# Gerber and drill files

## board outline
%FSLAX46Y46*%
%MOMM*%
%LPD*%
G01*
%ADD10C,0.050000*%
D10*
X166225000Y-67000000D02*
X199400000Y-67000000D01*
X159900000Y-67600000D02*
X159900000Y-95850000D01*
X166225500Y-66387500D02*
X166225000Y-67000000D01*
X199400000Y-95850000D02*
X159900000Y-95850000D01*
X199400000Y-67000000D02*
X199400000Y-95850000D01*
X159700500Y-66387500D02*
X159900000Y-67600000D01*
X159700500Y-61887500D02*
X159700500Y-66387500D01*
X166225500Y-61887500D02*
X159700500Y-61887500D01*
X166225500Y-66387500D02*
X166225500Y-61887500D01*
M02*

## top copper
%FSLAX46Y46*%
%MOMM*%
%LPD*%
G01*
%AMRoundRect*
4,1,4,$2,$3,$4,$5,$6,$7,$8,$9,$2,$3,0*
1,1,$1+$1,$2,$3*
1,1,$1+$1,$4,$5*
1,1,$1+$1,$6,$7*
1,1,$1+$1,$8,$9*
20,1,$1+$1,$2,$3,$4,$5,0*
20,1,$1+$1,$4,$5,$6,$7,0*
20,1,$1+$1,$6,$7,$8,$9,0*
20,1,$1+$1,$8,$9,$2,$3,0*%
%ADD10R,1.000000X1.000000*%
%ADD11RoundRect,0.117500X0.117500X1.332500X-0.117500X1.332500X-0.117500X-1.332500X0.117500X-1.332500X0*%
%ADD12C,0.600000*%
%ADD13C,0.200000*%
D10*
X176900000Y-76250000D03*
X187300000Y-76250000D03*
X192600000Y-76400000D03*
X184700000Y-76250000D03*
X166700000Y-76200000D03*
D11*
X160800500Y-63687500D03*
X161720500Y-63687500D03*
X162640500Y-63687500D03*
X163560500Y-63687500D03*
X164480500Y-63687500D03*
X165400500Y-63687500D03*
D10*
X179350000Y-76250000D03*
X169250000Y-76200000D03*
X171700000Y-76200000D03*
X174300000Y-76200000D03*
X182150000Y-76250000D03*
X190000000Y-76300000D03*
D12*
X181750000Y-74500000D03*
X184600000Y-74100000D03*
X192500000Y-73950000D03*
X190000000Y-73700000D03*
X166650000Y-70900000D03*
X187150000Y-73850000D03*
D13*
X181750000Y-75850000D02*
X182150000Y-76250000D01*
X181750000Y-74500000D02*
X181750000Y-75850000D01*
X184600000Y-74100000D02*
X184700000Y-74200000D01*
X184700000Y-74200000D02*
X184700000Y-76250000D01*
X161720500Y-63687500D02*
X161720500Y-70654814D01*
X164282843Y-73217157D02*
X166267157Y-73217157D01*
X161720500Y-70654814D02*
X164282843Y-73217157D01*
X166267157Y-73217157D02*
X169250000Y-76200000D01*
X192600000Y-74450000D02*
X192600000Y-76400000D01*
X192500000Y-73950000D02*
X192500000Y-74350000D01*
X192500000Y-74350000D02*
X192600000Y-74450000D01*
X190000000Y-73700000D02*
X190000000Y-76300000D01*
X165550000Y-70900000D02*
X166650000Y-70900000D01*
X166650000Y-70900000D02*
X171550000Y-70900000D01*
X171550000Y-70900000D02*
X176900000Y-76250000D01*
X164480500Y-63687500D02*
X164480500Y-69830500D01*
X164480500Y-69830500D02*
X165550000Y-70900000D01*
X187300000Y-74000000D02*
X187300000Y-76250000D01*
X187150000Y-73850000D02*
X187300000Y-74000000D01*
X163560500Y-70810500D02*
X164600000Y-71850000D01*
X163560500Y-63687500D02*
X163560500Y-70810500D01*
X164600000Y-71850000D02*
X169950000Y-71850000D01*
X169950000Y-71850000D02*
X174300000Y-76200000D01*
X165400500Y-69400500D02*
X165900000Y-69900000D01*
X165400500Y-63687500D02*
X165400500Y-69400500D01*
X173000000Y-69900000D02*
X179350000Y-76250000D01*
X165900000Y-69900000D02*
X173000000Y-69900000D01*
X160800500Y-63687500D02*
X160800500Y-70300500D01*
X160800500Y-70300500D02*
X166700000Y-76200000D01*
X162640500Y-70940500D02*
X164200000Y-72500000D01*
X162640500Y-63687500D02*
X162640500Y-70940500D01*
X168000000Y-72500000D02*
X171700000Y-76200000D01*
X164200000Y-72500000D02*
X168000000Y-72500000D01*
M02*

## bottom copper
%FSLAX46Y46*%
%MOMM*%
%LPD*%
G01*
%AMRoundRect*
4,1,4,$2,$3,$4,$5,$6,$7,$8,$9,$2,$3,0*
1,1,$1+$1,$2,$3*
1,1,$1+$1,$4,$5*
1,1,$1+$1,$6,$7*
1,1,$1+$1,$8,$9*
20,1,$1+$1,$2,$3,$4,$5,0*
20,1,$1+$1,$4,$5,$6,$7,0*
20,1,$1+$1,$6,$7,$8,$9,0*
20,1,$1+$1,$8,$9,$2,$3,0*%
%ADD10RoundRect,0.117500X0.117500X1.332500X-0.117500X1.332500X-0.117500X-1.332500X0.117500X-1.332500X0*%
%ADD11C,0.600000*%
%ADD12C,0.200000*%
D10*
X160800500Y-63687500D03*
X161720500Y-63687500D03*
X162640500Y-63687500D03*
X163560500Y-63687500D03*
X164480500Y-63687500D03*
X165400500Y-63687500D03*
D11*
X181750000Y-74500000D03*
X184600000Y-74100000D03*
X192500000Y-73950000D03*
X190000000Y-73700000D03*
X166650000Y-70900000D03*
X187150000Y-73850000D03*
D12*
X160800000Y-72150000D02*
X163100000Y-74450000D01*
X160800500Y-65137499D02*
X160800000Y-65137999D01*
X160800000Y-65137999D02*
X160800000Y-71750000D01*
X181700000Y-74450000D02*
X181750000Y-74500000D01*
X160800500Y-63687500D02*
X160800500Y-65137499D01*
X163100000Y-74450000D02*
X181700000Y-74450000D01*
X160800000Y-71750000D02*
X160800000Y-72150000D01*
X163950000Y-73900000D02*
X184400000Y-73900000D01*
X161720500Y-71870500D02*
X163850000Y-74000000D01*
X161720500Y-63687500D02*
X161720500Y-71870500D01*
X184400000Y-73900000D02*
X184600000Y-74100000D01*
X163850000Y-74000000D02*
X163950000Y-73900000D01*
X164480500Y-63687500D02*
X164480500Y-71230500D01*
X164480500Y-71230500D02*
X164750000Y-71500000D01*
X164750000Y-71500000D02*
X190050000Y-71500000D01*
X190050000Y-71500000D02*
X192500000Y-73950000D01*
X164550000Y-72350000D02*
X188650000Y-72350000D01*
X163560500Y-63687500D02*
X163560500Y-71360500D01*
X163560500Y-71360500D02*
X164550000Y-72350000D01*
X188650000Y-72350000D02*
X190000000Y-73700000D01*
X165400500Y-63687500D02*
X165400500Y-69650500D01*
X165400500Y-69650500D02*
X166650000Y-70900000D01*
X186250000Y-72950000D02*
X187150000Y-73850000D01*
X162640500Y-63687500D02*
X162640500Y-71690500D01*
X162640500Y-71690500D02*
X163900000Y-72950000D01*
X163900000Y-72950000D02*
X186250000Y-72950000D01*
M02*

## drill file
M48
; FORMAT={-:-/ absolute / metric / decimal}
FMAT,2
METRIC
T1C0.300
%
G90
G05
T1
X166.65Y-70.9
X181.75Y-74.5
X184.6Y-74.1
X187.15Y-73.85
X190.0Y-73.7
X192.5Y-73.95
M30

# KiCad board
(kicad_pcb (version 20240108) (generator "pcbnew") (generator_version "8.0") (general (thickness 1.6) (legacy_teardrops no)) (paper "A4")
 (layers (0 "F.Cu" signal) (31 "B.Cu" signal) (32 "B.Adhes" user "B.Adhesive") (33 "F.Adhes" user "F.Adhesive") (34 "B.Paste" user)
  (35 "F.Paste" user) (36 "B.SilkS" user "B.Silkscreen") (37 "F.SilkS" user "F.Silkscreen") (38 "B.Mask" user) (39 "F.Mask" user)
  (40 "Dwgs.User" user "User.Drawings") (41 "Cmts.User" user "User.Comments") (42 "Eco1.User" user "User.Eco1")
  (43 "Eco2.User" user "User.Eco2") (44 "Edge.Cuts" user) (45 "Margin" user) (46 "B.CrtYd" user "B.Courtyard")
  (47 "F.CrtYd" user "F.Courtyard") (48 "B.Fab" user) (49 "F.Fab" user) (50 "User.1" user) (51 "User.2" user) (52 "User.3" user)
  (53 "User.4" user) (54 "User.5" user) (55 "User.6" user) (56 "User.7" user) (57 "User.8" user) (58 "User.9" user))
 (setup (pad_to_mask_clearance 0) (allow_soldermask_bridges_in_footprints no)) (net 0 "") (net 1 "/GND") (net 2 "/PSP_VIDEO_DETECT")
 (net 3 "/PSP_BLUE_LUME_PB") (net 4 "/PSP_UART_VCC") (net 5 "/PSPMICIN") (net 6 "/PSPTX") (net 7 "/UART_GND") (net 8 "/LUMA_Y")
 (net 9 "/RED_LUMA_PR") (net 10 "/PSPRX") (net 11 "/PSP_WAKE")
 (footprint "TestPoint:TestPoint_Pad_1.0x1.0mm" (layer "F.Cu") (at 176.9 76.25)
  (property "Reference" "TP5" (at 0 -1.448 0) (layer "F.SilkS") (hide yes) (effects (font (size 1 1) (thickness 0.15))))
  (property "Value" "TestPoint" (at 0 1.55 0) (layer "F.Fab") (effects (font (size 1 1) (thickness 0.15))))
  (pad "1" smd rect (at 0 0) (size 1 1) (layers "F.Cu" "F.Mask") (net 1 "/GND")))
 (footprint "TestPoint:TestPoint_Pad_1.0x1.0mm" (layer "F.Cu") (at 187.3 76.25)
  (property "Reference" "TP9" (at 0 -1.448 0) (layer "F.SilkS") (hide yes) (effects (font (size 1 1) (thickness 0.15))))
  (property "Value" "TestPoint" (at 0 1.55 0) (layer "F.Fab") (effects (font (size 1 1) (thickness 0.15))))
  (pad "1" smd rect (at 0 0) (size 1 1) (layers "F.Cu" "F.Mask") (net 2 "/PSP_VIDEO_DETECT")))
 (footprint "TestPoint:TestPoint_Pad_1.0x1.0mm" (layer "F.Cu") (at 192.6 76.4)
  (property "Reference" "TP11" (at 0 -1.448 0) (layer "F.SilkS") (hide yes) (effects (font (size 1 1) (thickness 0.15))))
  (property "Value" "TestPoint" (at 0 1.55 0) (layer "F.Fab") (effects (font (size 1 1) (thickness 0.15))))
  (pad "1" smd rect (at 0 0) (size 1 1) (layers "F.Cu" "F.Mask") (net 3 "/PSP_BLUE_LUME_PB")))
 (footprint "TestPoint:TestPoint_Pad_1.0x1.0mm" (layer "F.Cu") (at 184.7 76.25)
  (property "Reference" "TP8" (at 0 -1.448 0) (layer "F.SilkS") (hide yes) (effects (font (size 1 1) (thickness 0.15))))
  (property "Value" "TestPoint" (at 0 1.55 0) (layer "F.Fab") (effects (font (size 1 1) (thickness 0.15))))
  (pad "1" smd rect (at 0 0) (size 1 1) (layers "F.Cu" "F.Mask") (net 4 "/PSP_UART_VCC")))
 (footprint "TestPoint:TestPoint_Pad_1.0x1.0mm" (layer "F.Cu") (at 166.7 76.2)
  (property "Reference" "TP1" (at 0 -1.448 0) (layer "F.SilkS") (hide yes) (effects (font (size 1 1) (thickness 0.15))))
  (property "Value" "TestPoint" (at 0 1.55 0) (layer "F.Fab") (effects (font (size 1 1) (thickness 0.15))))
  (pad "1" smd rect (at 0 0) (size 1 1) (layers "F.Cu" "F.Mask") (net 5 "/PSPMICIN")))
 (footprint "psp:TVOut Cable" (layer "F.Cu") (at 168.8255 70.9875)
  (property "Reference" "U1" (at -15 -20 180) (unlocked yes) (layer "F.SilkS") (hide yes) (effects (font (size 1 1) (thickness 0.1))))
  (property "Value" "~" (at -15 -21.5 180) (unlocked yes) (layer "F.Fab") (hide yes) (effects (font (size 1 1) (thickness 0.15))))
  (fp_line (start -9.125 -9.1) (end -9.125 -4.6) (stroke (width 0.05) (type default)) (layer "Edge.Cuts"))
  (fp_line (start -2.6 -9.1) (end -9.125 -9.1) (stroke (width 0.05) (type default)) (layer "Edge.Cuts"))
  (fp_line (start -2.6 -4.6) (end -2.6 -9.1) (stroke (width 0.05) (type default)) (layer "Edge.Cuts"))
  (pad "1" smd roundrect (at -8.025 -7.3 180) (size 0.47 2.9) (layers "F.Cu" "F.Paste" "F.Mask") (roundrect_rratio 0.25) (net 5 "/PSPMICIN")
   (thermal_bridge_angle 45))
  (pad "2" smd roundrect (at -7.105 -7.3 180) (size 0.47 2.9) (layers "F.Cu" "F.Paste" "F.Mask") (roundrect_rratio 0.25) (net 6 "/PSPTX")
   (thermal_bridge_angle 45))
  (pad "3" smd roundrect (at -6.185 -7.3 180) (size 0.47 2.9) (layers "F.Cu" "F.Paste" "F.Mask") (roundrect_rratio 0.25) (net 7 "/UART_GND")
   (thermal_bridge_angle 45))
  (pad "4" smd roundrect (at -5.265 -7.3 180) (size 0.47 2.9) (layers "F.Cu" "F.Paste" "F.Mask") (roundrect_rratio 0.25) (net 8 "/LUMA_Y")
   (thermal_bridge_angle 45))
  (pad "5" smd roundrect (at -4.345 -7.3 180) (size 0.47 2.9) (layers "F.Cu" "F.Paste" "F.Mask") (roundrect_rratio 0.25) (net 1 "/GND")
   (thermal_bridge_angle 45))
  (pad "6" smd roundrect (at -3.425 -7.3 180) (size 0.47 2.9) (layers "F.Cu" "F.Paste" "F.Mask") (roundrect_rratio 0.25)
   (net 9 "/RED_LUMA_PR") (thermal_bridge_angle 45))
  (pad "7" smd roundrect (at -8.025 -7.3 180) (size 0.47 2.9) (layers "B.Cu" "B.Paste" "B.Mask") (roundrect_rratio 0.25) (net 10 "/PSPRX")
   (thermal_bridge_angle 45))
  (pad "8" smd roundrect (at -7.105 -7.3 180) (size 0.47 2.9) (layers "B.Cu" "B.Paste" "B.Mask") (roundrect_rratio 0.25)
   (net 4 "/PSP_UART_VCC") (thermal_bridge_angle 45))
  (pad "9" smd roundrect (at -6.185 -7.3 180) (size 0.47 2.9) (layers "B.Cu" "B.Paste" "B.Mask") (roundrect_rratio 0.25)
   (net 2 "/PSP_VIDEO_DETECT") (thermal_bridge_angle 45))
  (pad "10" smd roundrect (at -5.265 -7.3 180) (size 0.47 2.9) (layers "B.Cu" "B.Paste" "B.Mask") (roundrect_rratio 0.25)
   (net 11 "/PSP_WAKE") (thermal_bridge_angle 45))
  (pad "11" smd roundrect (at -4.345 -7.3 180) (size 0.47 2.9) (layers "B.Cu" "B.Paste" "B.Mask") (roundrect_rratio 0.25)
   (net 3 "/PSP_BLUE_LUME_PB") (thermal_bridge_angle 45))
  (pad "12" smd roundrect (at -3.425 -7.3 180) (size 0.47 2.9) (layers "B.Cu" "B.Paste" "B.Mask") (roundrect_rratio 0.25) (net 1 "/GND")
   (thermal_bridge_angle 45)))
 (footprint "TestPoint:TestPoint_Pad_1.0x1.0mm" (layer "F.Cu") (at 179.35 76.25)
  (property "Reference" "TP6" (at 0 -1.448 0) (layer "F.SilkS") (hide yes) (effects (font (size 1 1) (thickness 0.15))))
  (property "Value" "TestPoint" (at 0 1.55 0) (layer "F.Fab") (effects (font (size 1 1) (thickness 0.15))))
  (pad "1" smd rect (at 0 0) (size 1 1) (layers "F.Cu" "F.Mask") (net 9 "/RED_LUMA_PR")))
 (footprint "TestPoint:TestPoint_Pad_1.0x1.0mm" (layer "F.Cu") (at 169.25 76.2)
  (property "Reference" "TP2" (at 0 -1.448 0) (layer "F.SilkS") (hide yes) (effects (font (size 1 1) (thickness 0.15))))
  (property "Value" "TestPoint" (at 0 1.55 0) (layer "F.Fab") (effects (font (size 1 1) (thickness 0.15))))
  (pad "1" smd rect (at 0 0) (size 1 1) (layers "F.Cu" "F.Mask") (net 6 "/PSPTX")))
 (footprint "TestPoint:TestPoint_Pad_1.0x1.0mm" (layer "F.Cu") (at 171.7 76.2)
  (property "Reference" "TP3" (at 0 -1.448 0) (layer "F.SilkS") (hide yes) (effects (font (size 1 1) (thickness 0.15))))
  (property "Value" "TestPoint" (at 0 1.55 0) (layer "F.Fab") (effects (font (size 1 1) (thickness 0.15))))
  (pad "1" smd rect (at 0 0) (size 1 1) (layers "F.Cu" "F.Mask") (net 7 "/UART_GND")))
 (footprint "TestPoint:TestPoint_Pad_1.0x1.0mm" (layer "F.Cu") (at 174.3 76.2)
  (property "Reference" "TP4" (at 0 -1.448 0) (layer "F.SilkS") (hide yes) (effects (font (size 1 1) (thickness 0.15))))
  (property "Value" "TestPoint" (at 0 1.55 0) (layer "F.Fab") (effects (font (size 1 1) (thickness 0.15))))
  (pad "1" smd rect (at 0 0) (size 1 1) (layers "F.Cu" "F.Mask") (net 8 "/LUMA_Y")))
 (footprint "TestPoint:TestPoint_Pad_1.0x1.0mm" (layer "F.Cu") (at 182.15 76.25)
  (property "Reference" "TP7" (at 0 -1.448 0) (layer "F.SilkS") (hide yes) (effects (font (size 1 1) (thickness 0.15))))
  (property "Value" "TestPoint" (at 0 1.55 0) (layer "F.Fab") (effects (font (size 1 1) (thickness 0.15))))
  (pad "1" smd rect (at 0 0) (size 1 1) (layers "F.Cu" "F.Mask") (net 10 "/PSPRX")))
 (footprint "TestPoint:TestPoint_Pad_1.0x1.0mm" (layer "F.Cu") (at 190 76.3)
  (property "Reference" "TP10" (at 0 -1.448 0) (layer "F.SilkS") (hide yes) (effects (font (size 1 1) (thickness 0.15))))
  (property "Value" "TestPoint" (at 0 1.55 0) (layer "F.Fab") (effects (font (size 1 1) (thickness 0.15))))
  (pad "1" smd rect (at 0 0) (size 1 1) (layers "F.Cu" "F.Mask") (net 11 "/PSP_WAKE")))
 (gr_line (start 166.225 67) (end 199.4 67) (stroke (width 0.05) (type default)) (layer "Edge.Cuts"))
 (gr_line (start 159.9 67.6) (end 159.9 95.85) (stroke (width 0.05) (type default)) (layer "Edge.Cuts"))
 (gr_line (start 166.2255 66.3875) (end 166.225 67) (stroke (width 0.05) (type default)) (layer "Edge.Cuts"))
 (gr_line (start 199.4 95.85) (end 159.9 95.85) (stroke (width 0.05) (type default)) (layer "Edge.Cuts"))
 (gr_line (start 199.4 67) (end 199.4 95.85) (stroke (width 0.05) (type default)) (layer "Edge.Cuts"))
 (gr_line (start 159.7005 66.3875) (end 159.9 67.6) (stroke (width 0.05) (type default)) (layer "Edge.Cuts"))
 (segment (start 181.75 75.85) (end 182.15 76.25) (width 0.2) (layer "F.Cu") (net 10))
 (segment (start 181.75 74.5) (end 181.75 75.85) (width 0.2) (layer "F.Cu") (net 10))
 (via (at 181.75 74.5) (size 0.6) (drill 0.3) (layers "F.Cu" "B.Cu") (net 10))
 (segment (start 160.8 72.15) (end 163.1 74.45) (width 0.2) (layer "B.Cu") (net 10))
 (segment (start 160.8005 65.137499) (end 160.8 65.137999) (width 0.2) (layer "B.Cu") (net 10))
 (segment (start 160.8 65.137999) (end 160.8 71.75) (width 0.2) (layer "B.Cu") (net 10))
 (segment (start 181.7 74.45) (end 181.75 74.5) (width 0.2) (layer "B.Cu") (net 10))
 (segment (start 160.8005 63.6875) (end 160.8005 65.137499) (width 0.2) (layer "B.Cu") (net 10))
 (segment (start 163.1 74.45) (end 181.7 74.45) (width 0.2) (layer "B.Cu") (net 10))
 (segment (start 160.8 71.75) (end 160.8 72.15) (width 0.2) (layer "B.Cu") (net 10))
 (segment (start 184.6 74.1) (end 184.7 74.2) (width 0.2) (layer "F.Cu") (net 4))
 (segment (start 184.7 74.2) (end 184.7 76.25) (width 0.2) (layer "F.Cu") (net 4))
 (via (at 184.6 74.1) (size 0.6) (drill 0.3) (layers "F.Cu" "B.Cu") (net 4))
 (segment (start 163.95 73.9) (end 184.4 73.9) (width 0.2) (layer "B.Cu") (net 4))
 (segment (start 161.7205 71.8705) (end 163.85 74) (width 0.2) (layer "B.Cu") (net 4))
 (segment (start 161.7205 63.6875) (end 161.7205 71.8705) (width 0.2) (layer "B.Cu") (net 4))
 (segment (start 184.4 73.9) (end 184.6 74.1) (width 0.2) (layer "B.Cu") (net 4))
 (segment (start 163.85 74) (end 163.95 73.9) (width 0.2) (layer "B.Cu") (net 4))
 (segment (start 161.7205 63.6875) (end 161.7205 70.654814) (width 0.2) (layer "F.Cu") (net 6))
 (segment (start 164.282843 73.217157) (end 166.267157 73.217157) (width 0.2) (layer "F.Cu") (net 6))
 (segment (start 161.7205 70.654814) (end 164.282843 73.217157) (width 0.2) (layer "F.Cu") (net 6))
 (segment (start 166.267157 73.217157) (end 169.25 76.2) (width 0.2) (layer "F.Cu") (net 6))
 (segment (start 192.6 74.45) (end 192.6 76.4) (width 0.2) (layer "F.Cu") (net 3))
 (segment (start 192.5 73.95) (end 192.5 74.35) (width 0.2) (layer "F.Cu") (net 3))
 (segment (start 192.5 74.35) (end 192.6 74.45) (width 0.2) (layer "F.Cu") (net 3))
 (via (at 192.5 73.95) (size 0.6) (drill 0.3) (layers "F.Cu" "B.Cu") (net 3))
 (segment (start 164.4805 63.6875) (end 164.4805 71.2305) (width 0.2) (layer "B.Cu") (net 3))
 (segment (start 164.4805 71.2305) (end 164.75 71.5) (width 0.2) (layer "B.Cu") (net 3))
 (segment (start 164.75 71.5) (end 190.05 71.5) (width 0.2) (layer "B.Cu") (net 3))
 (segment (start 190.05 71.5) (end 192.5 73.95) (width 0.2) (layer "B.Cu") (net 3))
 (segment (start 190 73.7) (end 190 76.3) (width 0.2) (layer "F.Cu") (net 11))
 (via (at 190 73.7) (size 0.6) (drill 0.3) (layers "F.Cu" "B.Cu") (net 11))
 (segment (start 164.55 72.35) (end 188.65 72.35) (width 0.2) (layer "B.Cu") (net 11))
 (segment (start 163.5605 63.6875) (end 163.5605 71.3605) (width 0.2) (layer "B.Cu") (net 11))
 (segment (start 163.5605 71.3605) (end 164.55 72.35) (width 0.2) (layer "B.Cu") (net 11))
 (segment (start 188.65 72.35) (end 190 73.7) (width 0.2) (layer "B.Cu") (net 11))
 (segment (start 165.55 70.9) (end 166.65 70.9) (width 0.2) (layer "F.Cu") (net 1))
 (segment (start 166.65 70.9) (end 171.55 70.9) (width 0.2) (layer "F.Cu") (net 1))
 (segment (start 171.55 70.9) (end 176.9 76.25) (width 0.2) (layer "F.Cu") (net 1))
 (segment (start 164.4805 63.6875) (end 164.4805 69.8305) (width 0.2) (layer "F.Cu") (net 1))
 (segment (start 164.4805 69.8305) (end 165.55 70.9) (width 0.2) (layer "F.Cu") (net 1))
 (via (at 166.65 70.9) (size 0.6) (drill 0.3) (layers "F.Cu" "B.Cu") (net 1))
 (segment (start 165.4005 63.6875) (end 165.4005 69.6505) (width 0.2) (layer "B.Cu") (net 1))
 (segment (start 165.4005 69.6505) (end 166.65 70.9) (width 0.2) (layer "B.Cu") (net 1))
 (segment (start 187.3 74) (end 187.3 76.25) (width 0.2) (layer "F.Cu") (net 2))
 (segment (start 187.15 73.85) (end 187.3 74) (width 0.2) (layer "F.Cu") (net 2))
 (via (at 187.15 73.85) (size 0.6) (drill 0.3) (layers "F.Cu" "B.Cu") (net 2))
 (segment (start 186.25 72.95) (end 187.15 73.85) (width 0.2) (layer "B.Cu") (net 2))
 (segment (start 162.6405 63.6875) (end 162.6405 71.6905) (width 0.2) (layer "B.Cu") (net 2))
 (segment (start 162.6405 71.6905) (end 163.9 72.95) (width 0.2) (layer "B.Cu") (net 2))
 (segment (start 163.9 72.95) (end 186.25 72.95) (width 0.2) (layer "B.Cu") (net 2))
 (segment (start 163.5605 70.8105) (end 164.6 71.85) (width 0.2) (layer "F.Cu") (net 8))
 (segment (start 163.5605 63.6875) (end 163.5605 70.8105) (width 0.2) (layer "F.Cu") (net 8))
 (segment (start 164.6 71.85) (end 169.95 71.85) (width 0.2) (layer "F.Cu") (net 8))
 (segment (start 169.95 71.85) (end 174.3 76.2) (width 0.2) (layer "F.Cu") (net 8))
 (segment (start 165.4005 69.4005) (end 165.9 69.9) (width 0.2) (layer "F.Cu") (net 9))
 (segment (start 165.4005 63.6875) (end 165.4005 69.4005) (width 0.2) (layer "F.Cu") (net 9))
 (segment (start 173 69.9) (end 179.35 76.25) (width 0.2) (layer "F.Cu") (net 9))
 (segment (start 165.9 69.9) (end 173 69.9) (width 0.2) (layer "F.Cu") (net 9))
 (segment (start 160.8005 63.6875) (end 160.8005 70.3005) (width 0.2) (layer "F.Cu") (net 5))
 (segment (start 160.8005 70.3005) (end 166.7 76.2) (width 0.2) (layer "F.Cu") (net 5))
 (segment (start 162.6405 70.9405) (end 164.2 72.5) (width 0.2) (layer "F.Cu") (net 7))
 (segment (start 162.6405 63.6875) (end 162.6405 70.9405) (width 0.2) (layer "F.Cu") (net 7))
 (segment (start 168 72.5) (end 171.7 76.2) (width 0.2) (layer "F.Cu") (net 7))
 (segment (start 164.2 72.5) (end 168 72.5) (width 0.2) (layer "F.Cu") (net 7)))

